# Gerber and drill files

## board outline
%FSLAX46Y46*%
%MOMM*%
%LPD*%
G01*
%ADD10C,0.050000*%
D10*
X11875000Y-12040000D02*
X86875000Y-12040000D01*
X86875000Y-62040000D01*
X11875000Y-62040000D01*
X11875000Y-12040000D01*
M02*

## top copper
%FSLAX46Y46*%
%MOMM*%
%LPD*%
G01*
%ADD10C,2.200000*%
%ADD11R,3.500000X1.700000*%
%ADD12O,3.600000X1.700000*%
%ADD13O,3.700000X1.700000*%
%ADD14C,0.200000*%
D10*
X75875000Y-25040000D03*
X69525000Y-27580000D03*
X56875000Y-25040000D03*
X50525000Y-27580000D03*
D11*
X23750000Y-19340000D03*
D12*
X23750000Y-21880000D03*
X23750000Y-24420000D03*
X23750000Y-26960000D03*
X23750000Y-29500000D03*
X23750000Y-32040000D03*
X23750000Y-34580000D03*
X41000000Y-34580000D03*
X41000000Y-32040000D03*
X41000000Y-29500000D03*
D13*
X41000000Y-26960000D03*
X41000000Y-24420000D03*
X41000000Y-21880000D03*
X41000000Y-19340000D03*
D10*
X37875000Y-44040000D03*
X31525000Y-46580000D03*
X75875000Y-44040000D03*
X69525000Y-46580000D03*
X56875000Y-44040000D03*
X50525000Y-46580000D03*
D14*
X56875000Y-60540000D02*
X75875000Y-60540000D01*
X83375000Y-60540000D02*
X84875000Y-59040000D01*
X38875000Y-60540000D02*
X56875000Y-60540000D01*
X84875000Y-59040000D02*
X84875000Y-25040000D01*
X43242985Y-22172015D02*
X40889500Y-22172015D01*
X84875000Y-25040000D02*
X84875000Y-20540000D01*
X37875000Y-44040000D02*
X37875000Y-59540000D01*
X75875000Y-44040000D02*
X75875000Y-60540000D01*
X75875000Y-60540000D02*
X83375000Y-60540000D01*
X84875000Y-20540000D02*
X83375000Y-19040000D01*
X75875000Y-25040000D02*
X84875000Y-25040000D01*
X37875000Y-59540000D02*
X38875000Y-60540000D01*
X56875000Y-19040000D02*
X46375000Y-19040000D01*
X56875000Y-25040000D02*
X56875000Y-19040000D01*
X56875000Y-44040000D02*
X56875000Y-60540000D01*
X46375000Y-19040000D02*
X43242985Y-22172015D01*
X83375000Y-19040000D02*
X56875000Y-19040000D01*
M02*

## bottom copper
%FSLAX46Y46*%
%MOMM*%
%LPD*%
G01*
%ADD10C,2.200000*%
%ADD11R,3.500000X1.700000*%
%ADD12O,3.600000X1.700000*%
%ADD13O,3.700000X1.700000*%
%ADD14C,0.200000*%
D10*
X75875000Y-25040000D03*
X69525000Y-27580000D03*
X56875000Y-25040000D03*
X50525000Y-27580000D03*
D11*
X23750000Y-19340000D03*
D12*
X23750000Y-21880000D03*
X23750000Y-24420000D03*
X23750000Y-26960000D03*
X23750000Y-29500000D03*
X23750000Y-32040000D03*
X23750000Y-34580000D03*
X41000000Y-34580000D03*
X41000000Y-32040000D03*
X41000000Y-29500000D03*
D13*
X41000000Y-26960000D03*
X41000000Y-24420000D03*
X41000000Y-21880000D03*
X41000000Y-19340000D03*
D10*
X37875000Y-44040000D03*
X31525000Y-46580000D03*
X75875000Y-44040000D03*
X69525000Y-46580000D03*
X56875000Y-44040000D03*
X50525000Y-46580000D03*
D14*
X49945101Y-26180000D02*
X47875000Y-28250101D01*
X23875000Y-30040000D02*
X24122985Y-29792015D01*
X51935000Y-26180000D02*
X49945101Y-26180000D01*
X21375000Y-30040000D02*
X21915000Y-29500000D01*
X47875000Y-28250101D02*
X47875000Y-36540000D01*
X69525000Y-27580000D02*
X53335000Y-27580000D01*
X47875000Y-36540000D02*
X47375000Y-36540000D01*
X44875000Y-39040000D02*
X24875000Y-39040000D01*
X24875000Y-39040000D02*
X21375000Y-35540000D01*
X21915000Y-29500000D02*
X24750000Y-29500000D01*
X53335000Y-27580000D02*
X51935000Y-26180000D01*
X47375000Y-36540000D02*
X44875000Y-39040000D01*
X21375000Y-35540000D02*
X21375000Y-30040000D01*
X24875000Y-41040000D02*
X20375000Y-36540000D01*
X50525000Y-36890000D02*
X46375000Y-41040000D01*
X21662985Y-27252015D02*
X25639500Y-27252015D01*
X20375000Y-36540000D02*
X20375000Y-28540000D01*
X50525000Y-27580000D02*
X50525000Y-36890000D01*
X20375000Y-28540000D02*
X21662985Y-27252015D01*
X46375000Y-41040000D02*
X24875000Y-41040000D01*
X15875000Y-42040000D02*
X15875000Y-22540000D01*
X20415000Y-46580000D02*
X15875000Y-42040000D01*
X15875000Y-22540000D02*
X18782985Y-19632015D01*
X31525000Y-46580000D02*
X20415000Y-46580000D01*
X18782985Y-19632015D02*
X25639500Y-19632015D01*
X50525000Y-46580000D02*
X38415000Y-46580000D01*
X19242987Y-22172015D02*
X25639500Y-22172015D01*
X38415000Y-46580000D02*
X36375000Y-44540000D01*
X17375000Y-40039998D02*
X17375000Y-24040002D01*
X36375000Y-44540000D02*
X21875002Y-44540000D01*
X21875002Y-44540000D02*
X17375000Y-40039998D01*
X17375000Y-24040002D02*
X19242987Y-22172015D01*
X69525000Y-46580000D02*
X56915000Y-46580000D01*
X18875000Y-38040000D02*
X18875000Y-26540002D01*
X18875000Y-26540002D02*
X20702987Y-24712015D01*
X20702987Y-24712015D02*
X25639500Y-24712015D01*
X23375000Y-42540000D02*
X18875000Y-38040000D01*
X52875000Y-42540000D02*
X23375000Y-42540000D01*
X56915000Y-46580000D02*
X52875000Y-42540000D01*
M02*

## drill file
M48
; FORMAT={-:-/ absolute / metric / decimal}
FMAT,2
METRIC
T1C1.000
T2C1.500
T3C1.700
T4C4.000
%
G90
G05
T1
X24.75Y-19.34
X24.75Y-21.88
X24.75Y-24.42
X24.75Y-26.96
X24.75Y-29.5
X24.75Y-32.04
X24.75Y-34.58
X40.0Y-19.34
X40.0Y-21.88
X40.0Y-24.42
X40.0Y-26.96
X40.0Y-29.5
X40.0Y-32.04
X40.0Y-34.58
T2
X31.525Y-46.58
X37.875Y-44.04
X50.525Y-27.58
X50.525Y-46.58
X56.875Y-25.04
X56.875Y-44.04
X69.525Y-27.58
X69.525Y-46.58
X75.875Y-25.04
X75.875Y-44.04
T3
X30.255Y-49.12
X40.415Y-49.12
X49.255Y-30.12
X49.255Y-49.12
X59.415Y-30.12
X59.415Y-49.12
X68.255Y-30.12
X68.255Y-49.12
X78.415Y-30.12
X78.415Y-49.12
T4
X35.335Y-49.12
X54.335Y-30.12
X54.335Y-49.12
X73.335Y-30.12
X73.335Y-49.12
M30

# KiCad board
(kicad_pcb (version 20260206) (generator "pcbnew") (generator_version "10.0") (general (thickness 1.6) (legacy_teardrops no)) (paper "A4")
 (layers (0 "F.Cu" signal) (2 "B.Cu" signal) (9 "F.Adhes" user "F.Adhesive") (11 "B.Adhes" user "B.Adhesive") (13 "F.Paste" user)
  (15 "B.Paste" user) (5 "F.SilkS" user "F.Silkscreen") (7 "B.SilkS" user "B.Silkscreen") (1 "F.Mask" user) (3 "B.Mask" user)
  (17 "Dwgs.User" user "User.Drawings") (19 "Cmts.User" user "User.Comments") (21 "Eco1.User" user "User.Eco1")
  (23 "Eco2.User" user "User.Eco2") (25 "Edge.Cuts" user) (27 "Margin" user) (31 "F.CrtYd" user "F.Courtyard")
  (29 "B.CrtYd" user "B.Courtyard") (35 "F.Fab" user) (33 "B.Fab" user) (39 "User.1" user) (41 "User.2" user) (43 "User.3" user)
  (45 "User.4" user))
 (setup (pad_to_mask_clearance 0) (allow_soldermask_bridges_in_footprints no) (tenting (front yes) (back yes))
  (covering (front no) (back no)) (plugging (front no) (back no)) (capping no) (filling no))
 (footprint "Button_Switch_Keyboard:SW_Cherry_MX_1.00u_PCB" (layer "F.Cu") (at 75.875 25.04)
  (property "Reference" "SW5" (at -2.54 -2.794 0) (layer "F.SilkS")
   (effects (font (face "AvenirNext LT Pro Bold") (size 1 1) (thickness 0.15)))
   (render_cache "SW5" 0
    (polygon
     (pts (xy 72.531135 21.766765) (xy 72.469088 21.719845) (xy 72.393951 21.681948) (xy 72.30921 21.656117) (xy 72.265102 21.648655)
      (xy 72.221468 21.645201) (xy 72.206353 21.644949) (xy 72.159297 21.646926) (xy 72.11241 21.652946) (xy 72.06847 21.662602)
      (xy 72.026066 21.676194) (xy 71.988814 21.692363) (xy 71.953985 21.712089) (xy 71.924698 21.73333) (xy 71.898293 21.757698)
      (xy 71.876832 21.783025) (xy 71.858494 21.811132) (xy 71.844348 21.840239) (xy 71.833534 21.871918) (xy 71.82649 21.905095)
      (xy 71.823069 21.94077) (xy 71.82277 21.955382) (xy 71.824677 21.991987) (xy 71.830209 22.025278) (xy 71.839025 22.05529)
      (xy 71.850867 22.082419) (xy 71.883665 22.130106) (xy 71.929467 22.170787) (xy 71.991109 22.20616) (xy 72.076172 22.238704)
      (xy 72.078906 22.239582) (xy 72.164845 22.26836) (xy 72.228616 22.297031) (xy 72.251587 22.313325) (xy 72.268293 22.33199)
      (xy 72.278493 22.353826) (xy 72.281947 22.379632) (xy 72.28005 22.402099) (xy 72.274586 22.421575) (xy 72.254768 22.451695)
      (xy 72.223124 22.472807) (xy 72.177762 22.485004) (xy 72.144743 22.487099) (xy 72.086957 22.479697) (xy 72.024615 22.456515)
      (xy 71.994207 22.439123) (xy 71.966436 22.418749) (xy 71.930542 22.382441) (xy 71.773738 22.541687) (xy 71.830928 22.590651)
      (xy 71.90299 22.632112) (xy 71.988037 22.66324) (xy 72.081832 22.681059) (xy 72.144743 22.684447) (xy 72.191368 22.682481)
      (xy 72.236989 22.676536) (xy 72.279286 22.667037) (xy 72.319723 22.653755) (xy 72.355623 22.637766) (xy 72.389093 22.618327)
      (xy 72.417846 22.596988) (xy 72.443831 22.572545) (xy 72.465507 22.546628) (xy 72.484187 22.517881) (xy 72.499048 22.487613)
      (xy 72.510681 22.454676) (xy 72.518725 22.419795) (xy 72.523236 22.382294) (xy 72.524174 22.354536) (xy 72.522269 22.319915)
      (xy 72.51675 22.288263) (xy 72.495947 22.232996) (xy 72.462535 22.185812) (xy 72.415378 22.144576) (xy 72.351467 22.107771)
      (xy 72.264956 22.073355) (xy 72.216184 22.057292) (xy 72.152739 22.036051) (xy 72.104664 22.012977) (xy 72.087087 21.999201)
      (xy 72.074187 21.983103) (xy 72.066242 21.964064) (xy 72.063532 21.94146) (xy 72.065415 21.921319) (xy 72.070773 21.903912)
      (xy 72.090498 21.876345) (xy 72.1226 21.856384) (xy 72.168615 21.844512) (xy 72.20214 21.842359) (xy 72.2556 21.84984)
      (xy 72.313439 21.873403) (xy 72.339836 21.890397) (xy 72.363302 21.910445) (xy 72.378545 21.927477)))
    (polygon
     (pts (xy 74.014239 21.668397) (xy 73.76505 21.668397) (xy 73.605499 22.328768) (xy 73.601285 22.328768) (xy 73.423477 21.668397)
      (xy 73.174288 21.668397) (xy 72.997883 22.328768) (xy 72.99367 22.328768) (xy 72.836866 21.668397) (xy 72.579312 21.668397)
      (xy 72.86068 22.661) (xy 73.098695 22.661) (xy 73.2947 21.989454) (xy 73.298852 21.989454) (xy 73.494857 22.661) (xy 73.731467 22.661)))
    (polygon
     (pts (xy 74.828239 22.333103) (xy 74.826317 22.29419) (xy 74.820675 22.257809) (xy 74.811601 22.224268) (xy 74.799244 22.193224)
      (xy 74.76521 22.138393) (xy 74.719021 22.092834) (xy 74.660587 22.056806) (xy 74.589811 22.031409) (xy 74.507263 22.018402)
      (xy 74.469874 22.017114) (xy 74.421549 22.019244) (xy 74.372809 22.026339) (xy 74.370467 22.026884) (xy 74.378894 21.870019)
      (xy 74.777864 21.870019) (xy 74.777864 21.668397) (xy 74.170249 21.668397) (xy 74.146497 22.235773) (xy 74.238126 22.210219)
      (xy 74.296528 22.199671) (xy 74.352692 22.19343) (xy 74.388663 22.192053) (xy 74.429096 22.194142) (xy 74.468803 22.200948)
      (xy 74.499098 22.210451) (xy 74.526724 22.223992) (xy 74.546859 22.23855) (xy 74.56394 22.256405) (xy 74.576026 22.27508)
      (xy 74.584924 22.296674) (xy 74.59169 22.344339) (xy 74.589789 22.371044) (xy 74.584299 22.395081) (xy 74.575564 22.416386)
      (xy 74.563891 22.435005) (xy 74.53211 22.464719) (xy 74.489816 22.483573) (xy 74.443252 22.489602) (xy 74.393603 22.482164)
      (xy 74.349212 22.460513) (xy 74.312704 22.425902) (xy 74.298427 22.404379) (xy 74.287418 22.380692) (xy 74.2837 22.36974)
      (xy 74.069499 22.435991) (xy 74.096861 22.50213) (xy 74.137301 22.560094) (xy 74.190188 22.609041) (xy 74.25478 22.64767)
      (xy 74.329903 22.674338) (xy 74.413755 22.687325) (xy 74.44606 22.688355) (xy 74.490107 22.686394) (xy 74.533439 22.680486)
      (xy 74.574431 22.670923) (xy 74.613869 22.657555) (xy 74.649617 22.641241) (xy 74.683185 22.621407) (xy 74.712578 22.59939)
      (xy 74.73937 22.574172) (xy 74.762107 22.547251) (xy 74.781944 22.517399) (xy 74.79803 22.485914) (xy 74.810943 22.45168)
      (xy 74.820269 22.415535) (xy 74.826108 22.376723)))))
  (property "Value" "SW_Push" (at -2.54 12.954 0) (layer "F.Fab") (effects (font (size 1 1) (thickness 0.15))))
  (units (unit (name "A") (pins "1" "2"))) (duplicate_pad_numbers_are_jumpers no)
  (pad "" np_thru_hole circle (at -7.62 5.08) (size 1.7 1.7) (drill 1.7) (layers "*.Cu" "*.Mask"))
  (pad "" np_thru_hole circle (at -2.54 5.08) (size 4 4) (drill 4) (layers "*.Cu" "*.Mask"))
  (pad "" np_thru_hole circle (at 2.54 5.08) (size 1.7 1.7) (drill 1.7) (layers "*.Cu" "*.Mask"))
  (pad "1" thru_hole circle (at 0 0) (size 2.2 2.2) (drill 1.5) (layers "*.Cu" "*.Mask") (remove_unused_layers no) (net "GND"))
  (pad "2" thru_hole circle (at -6.35 2.54) (size 2.2 2.2) (drill 1.5) (layers "*.Cu" "*.Mask") (remove_unused_layers no)
   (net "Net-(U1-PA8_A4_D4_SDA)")))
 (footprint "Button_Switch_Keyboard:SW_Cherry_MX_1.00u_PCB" (layer "F.Cu") (at 56.875 25.04)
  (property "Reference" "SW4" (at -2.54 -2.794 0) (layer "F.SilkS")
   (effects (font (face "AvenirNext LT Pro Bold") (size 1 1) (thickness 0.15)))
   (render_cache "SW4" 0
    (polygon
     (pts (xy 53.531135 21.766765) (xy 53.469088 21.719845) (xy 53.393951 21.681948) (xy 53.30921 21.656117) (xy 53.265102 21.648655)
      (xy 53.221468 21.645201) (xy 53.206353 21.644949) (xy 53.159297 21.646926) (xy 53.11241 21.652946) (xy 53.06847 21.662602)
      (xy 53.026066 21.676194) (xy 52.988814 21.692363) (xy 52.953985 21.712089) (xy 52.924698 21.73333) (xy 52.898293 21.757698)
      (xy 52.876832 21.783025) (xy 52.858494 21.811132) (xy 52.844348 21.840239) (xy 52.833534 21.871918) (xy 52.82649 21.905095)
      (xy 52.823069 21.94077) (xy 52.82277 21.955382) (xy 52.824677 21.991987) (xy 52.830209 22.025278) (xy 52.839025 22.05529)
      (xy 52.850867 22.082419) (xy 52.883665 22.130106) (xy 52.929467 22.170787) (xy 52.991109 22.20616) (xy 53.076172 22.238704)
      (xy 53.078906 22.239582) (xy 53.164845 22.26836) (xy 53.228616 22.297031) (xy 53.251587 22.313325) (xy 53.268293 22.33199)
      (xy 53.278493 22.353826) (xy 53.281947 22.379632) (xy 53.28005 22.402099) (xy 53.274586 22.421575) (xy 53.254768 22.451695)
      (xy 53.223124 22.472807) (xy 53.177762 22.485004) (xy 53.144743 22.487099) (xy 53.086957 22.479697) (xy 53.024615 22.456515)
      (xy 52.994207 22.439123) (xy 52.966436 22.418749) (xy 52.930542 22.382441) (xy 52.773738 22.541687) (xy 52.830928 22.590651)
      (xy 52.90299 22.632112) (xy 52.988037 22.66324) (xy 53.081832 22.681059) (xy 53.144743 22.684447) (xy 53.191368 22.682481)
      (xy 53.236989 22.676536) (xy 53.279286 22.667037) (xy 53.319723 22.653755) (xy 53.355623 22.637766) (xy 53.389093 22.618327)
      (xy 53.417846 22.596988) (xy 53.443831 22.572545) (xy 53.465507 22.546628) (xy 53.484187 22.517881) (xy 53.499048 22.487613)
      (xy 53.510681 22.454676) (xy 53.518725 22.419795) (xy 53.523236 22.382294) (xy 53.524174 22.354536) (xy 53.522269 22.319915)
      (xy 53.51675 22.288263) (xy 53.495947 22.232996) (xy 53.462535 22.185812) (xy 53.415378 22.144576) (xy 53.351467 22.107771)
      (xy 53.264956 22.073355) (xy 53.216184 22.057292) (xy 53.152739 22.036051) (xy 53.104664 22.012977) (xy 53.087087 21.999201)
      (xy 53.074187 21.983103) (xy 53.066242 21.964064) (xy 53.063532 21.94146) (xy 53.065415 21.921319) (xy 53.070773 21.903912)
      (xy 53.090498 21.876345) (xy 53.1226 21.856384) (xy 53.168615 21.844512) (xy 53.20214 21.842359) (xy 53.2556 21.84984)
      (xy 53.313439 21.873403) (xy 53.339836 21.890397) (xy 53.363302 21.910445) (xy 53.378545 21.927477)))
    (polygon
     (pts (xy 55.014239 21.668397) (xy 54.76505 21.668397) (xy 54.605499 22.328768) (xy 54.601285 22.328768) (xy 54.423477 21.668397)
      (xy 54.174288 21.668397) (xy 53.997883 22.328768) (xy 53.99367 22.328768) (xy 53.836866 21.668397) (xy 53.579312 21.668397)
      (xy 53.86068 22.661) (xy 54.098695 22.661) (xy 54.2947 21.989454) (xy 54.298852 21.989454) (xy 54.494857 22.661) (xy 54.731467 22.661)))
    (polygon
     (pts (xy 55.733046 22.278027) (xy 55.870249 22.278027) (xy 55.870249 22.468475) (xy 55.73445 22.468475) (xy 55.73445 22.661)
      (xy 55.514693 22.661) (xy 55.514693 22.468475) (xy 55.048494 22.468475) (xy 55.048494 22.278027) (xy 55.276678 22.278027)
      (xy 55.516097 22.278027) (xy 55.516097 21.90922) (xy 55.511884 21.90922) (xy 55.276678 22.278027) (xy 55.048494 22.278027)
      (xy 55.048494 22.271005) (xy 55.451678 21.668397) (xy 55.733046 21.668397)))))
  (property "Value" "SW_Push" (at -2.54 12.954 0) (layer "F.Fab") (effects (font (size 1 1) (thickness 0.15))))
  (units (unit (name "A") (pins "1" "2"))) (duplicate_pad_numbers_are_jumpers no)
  (pad "" np_thru_hole circle (at -7.62 5.08) (size 1.7 1.7) (drill 1.7) (layers "*.Cu" "*.Mask"))
  (pad "" np_thru_hole circle (at -2.54 5.08) (size 4 4) (drill 4) (layers "*.Cu" "*.Mask"))
  (pad "" np_thru_hole circle (at 2.54 5.08) (size 1.7 1.7) (drill 1.7) (layers "*.Cu" "*.Mask"))
  (pad "1" thru_hole circle (at 0 0) (size 2.2 2.2) (drill 1.5) (layers "*.Cu" "*.Mask") (remove_unused_layers no) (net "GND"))
  (pad "2" thru_hole circle (at -6.35 2.54) (size 2.2 2.2) (drill 1.5) (layers "*.Cu" "*.Mask") (remove_unused_layers no)
   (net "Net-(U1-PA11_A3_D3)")))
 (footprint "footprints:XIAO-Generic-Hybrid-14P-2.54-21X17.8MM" (layer "F.Cu") (at 32.375 26.96)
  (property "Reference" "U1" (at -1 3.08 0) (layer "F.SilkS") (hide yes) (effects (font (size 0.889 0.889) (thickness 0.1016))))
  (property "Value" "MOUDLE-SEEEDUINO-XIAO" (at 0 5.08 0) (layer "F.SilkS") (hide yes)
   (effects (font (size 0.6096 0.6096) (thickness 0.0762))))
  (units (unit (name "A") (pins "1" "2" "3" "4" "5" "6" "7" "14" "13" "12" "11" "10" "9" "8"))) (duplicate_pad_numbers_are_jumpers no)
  (pad "1" thru_hole rect (at -7.625 -7.62) (size 3.5 1.7) (drill 1 (offset -1 0)) (layers "*.Cu" "*.Mask") (remove_unused_layers no)
   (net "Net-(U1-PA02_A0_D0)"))
  (pad "2" thru_hole oval (at -7.625 -5.08) (size 3.6 1.7) (drill 1 (offset -1 0)) (layers "*.Cu" "*.Mask") (remove_unused_layers no)
   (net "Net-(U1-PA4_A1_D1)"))
  (pad "3" thru_hole oval (at -7.625 -2.54) (size 3.6 1.7) (drill 1 (offset -1 0)) (layers "*.Cu" "*.Mask") (remove_unused_layers no)
   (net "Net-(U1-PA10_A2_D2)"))
  (pad "4" thru_hole oval (at -7.625 0) (size 3.6 1.7) (drill 1 (offset -1 0)) (layers "*.Cu" "*.Mask") (remove_unused_layers no)
   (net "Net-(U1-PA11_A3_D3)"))
  (pad "5" thru_hole oval (at -7.625 2.54) (size 3.6 1.7) (drill 1 (offset -1 0)) (layers "*.Cu" "*.Mask") (remove_unused_layers no)
   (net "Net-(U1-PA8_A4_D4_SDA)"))
  (pad "6" thru_hole oval (at -7.625 5.08 180) (size 3.6 1.7) (drill 1 (offset 1 0)) (layers "*.Cu" "*.Mask") (remove_unused_layers no)
   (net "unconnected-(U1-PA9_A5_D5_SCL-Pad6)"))
  (pad "7" thru_hole oval (at -7.625 7.62) (size 3.6 1.7) (drill 1 (offset -1 0)) (layers "*.Cu" "*.Mask") (remove_unused_layers no)
   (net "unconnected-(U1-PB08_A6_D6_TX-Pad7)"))
  (pad "8" thru_hole oval (at 7.625 7.62) (size 3.6 1.7) (drill 1 (offset 1 0)) (layers "*.Cu" "*.Mask") (remove_unused_layers no)
   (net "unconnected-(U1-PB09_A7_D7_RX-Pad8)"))
  (pad "9" thru_hole oval (at 7.625 5.08) (size 3.6 1.7) (drill 1 (offset 1 0)) (layers "*.Cu" "*.Mask") (remove_unused_layers no)
   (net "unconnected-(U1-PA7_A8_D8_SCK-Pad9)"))
  (pad "10" thru_hole oval (at 7.625 2.54) (size 3.6 1.7) (drill 1 (offset 1 0)) (layers "*.Cu" "*.Mask") (remove_unused_layers no)
   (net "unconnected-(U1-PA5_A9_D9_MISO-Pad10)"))
  (pad "11" thru_hole oval (at 7.625 0) (size 3.7 1.7) (drill 1 (offset 1 0)) (layers "*.Cu" "*.Mask") (remove_unused_layers no)
   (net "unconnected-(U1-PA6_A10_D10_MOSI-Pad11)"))
  (pad "12" thru_hole oval (at 7.625 -2.54) (size 3.7 1.7) (drill 1 (offset 1 0)) (layers "*.Cu" "*.Mask") (remove_unused_layers no)
   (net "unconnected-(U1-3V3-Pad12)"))
  (pad "13" thru_hole oval (at 7.625 -5.08) (size 3.7 1.7) (drill 1 (offset 1 0)) (layers "*.Cu" "*.Mask") (remove_unused_layers no)
   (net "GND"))
  (pad "14" thru_hole oval (at 7.625 -7.62) (size 3.7 1.7) (drill 1 (offset 1 0)) (layers "*.Cu" "*.Mask") (remove_unused_layers no)
   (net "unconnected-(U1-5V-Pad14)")))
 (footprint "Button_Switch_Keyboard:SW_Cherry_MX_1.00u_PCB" (layer "F.Cu") (at 37.875 44.04)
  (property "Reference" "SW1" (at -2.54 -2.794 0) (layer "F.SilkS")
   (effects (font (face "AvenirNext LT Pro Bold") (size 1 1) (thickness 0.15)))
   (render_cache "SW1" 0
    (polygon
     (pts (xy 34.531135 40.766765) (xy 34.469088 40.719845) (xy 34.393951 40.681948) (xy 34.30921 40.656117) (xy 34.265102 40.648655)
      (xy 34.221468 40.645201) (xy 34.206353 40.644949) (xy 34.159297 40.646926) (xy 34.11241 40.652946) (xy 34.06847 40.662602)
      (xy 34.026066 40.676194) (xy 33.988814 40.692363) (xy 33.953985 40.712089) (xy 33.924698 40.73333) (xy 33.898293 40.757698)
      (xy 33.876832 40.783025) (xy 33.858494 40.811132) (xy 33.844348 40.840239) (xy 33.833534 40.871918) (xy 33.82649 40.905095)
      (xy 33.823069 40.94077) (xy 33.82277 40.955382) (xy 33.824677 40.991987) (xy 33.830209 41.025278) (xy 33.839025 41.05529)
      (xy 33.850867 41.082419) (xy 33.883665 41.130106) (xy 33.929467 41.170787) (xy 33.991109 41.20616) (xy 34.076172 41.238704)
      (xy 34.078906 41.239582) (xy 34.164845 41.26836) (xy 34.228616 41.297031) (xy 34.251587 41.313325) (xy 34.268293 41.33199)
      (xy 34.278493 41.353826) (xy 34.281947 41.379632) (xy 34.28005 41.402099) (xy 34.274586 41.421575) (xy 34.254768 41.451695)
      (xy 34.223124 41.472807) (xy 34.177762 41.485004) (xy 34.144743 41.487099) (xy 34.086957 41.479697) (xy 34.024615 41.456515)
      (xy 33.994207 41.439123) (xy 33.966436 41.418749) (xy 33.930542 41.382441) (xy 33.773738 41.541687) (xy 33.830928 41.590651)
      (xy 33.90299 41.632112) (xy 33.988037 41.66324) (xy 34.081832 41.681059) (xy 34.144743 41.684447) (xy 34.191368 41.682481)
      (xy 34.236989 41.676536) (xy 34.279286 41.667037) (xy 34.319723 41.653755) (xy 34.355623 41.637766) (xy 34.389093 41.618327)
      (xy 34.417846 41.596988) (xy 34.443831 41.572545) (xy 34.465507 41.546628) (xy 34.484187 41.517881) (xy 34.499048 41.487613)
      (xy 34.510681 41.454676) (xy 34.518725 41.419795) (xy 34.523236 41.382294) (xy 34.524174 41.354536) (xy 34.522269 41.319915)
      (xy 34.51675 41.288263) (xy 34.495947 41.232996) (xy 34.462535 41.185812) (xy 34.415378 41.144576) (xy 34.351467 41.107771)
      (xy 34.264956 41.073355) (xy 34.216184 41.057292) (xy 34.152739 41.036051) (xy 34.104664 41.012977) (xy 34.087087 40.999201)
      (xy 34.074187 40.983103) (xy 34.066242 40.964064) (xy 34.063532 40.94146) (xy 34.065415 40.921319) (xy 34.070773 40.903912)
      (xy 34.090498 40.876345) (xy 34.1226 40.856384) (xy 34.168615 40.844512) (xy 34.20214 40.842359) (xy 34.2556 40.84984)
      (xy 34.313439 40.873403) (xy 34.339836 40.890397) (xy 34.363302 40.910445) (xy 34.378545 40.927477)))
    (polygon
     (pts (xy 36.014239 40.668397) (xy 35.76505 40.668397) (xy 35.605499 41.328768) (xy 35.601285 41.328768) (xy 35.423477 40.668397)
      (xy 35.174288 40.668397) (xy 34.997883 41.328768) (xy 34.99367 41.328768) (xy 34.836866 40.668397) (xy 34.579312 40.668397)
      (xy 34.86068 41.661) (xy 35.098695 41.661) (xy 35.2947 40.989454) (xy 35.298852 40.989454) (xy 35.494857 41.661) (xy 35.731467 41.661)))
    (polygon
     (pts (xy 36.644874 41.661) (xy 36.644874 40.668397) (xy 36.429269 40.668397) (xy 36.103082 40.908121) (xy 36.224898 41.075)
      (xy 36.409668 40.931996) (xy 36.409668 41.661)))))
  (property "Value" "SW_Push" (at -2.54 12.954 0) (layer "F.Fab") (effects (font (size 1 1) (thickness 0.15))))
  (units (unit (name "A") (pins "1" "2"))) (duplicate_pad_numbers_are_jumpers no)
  (pad "" np_thru_hole circle (at -7.62 5.08) (size 1.7 1.7) (drill 1.7) (layers "*.Cu" "*.Mask"))
  (pad "" np_thru_hole circle (at -2.54 5.08) (size 4 4) (drill 4) (layers "*.Cu" "*.Mask"))
  (pad "" np_thru_hole circle (at 2.54 5.08) (size 1.7 1.7) (drill 1.7) (layers "*.Cu" "*.Mask"))
  (pad "1" thru_hole circle (at 0 0) (size 2.2 2.2) (drill 1.5) (layers "*.Cu" "*.Mask") (remove_unused_layers no) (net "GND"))
  (pad "2" thru_hole circle (at -6.35 2.54) (size 2.2 2.2) (drill 1.5) (layers "*.Cu" "*.Mask") (remove_unused_layers no)
   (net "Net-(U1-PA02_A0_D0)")))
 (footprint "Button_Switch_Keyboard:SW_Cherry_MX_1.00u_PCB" (layer "F.Cu") (at 75.875 44.04)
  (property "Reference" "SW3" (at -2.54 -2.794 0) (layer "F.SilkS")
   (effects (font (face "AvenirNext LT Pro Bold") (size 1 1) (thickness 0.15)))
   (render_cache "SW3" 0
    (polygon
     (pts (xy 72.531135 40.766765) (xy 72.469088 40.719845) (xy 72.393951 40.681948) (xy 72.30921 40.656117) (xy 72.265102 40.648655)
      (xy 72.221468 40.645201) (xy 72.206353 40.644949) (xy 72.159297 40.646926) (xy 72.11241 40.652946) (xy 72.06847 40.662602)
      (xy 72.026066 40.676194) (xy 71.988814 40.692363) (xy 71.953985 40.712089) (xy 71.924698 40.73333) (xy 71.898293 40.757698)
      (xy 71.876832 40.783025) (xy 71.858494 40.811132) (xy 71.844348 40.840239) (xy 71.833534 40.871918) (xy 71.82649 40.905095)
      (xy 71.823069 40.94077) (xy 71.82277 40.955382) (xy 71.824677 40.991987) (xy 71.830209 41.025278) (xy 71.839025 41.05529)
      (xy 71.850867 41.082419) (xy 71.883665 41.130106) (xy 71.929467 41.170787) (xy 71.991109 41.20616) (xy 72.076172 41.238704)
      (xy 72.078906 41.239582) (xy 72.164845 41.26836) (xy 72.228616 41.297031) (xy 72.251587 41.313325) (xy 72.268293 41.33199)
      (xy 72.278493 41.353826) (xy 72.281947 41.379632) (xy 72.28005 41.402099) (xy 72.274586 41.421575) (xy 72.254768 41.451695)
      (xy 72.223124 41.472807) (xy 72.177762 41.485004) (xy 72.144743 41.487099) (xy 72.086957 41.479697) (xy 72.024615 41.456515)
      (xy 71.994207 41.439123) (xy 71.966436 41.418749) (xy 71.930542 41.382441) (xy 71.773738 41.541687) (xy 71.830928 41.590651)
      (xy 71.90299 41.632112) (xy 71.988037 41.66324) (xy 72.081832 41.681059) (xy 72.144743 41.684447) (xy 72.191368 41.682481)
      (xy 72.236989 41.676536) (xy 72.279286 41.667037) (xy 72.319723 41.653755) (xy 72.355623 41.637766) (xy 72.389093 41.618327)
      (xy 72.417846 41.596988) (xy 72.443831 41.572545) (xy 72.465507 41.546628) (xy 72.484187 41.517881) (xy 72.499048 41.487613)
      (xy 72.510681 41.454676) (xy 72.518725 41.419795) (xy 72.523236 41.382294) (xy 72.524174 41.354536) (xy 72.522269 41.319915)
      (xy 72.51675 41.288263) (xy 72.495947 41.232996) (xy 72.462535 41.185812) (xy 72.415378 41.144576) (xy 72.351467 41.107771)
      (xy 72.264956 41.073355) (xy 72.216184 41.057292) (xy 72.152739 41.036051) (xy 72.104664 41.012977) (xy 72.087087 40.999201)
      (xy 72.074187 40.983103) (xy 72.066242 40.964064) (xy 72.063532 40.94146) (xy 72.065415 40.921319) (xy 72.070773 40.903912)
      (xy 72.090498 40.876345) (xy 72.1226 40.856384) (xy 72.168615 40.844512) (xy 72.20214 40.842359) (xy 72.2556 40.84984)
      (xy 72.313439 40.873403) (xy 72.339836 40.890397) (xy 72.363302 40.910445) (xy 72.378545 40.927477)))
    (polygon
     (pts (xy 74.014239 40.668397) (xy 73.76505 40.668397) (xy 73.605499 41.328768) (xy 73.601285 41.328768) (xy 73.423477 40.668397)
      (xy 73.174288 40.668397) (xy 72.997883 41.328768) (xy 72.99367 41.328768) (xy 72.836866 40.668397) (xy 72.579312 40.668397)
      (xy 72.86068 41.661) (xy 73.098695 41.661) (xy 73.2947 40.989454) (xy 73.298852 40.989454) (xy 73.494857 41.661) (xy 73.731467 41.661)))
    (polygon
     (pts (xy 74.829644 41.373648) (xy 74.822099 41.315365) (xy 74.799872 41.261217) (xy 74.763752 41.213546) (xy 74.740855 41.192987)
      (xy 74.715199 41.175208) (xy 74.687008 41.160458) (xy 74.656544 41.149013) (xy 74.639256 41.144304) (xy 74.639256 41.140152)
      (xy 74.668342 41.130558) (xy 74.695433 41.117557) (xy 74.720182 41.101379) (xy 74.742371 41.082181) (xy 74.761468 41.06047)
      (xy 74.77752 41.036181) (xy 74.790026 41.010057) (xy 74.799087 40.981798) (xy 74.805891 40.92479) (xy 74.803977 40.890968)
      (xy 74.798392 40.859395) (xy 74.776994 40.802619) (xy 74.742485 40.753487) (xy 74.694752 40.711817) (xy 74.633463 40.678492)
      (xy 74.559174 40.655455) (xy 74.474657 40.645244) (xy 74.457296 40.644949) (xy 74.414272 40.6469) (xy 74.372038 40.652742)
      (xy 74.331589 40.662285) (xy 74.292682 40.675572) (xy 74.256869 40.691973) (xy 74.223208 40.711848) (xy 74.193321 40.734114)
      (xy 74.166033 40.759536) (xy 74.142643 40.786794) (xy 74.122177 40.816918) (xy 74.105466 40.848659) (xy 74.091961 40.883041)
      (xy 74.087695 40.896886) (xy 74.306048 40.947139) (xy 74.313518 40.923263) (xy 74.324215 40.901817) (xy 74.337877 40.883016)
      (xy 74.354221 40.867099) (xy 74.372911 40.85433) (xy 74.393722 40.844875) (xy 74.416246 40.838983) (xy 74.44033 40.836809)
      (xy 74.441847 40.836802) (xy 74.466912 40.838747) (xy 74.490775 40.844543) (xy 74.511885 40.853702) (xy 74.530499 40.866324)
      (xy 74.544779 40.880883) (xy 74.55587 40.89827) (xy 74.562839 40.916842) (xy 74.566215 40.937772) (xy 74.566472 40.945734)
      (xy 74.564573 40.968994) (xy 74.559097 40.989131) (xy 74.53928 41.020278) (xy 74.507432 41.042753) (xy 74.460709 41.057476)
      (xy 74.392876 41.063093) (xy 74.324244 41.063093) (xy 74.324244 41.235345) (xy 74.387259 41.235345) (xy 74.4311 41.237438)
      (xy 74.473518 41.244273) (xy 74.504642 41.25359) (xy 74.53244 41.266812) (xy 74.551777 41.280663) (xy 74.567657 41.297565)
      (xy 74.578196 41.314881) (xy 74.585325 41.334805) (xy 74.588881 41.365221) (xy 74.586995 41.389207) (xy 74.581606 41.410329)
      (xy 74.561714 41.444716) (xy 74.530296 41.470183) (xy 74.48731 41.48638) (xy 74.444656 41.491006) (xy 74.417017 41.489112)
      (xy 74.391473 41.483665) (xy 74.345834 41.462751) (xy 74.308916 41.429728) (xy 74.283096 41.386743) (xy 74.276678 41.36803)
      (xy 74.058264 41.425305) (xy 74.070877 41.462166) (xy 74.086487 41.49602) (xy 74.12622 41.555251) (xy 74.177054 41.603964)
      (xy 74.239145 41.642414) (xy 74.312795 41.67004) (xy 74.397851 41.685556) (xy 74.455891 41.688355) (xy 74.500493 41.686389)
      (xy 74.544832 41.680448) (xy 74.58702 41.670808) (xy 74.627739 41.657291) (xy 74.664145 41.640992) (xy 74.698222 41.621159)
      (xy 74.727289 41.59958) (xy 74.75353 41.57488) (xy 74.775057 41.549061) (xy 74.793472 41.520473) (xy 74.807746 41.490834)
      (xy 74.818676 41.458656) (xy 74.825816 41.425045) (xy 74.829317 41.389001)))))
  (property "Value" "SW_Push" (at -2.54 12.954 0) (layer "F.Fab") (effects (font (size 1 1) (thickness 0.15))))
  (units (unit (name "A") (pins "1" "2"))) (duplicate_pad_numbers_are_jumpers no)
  (pad "" np_thru_hole circle (at -7.62 5.08) (size 1.7 1.7) (drill 1.7) (layers "*.Cu" "*.Mask"))
  (pad "" np_thru_hole circle (at -2.54 5.08) (size 4 4) (drill 4) (layers "*.Cu" "*.Mask"))
  (pad "" np_thru_hole circle (at 2.54 5.08) (size 1.7 1.7) (drill 1.7) (layers "*.Cu" "*.Mask"))
  (pad "1" thru_hole circle (at 0 0) (size 2.2 2.2) (drill 1.5) (layers "*.Cu" "*.Mask") (remove_unused_layers no) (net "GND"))
  (pad "2" thru_hole circle (at -6.35 2.54) (size 2.2 2.2) (drill 1.5) (layers "*.Cu" "*.Mask") (remove_unused_layers no)
   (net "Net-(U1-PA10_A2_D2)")))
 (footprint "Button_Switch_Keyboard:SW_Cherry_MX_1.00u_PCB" (layer "F.Cu") (at 56.875 44.04)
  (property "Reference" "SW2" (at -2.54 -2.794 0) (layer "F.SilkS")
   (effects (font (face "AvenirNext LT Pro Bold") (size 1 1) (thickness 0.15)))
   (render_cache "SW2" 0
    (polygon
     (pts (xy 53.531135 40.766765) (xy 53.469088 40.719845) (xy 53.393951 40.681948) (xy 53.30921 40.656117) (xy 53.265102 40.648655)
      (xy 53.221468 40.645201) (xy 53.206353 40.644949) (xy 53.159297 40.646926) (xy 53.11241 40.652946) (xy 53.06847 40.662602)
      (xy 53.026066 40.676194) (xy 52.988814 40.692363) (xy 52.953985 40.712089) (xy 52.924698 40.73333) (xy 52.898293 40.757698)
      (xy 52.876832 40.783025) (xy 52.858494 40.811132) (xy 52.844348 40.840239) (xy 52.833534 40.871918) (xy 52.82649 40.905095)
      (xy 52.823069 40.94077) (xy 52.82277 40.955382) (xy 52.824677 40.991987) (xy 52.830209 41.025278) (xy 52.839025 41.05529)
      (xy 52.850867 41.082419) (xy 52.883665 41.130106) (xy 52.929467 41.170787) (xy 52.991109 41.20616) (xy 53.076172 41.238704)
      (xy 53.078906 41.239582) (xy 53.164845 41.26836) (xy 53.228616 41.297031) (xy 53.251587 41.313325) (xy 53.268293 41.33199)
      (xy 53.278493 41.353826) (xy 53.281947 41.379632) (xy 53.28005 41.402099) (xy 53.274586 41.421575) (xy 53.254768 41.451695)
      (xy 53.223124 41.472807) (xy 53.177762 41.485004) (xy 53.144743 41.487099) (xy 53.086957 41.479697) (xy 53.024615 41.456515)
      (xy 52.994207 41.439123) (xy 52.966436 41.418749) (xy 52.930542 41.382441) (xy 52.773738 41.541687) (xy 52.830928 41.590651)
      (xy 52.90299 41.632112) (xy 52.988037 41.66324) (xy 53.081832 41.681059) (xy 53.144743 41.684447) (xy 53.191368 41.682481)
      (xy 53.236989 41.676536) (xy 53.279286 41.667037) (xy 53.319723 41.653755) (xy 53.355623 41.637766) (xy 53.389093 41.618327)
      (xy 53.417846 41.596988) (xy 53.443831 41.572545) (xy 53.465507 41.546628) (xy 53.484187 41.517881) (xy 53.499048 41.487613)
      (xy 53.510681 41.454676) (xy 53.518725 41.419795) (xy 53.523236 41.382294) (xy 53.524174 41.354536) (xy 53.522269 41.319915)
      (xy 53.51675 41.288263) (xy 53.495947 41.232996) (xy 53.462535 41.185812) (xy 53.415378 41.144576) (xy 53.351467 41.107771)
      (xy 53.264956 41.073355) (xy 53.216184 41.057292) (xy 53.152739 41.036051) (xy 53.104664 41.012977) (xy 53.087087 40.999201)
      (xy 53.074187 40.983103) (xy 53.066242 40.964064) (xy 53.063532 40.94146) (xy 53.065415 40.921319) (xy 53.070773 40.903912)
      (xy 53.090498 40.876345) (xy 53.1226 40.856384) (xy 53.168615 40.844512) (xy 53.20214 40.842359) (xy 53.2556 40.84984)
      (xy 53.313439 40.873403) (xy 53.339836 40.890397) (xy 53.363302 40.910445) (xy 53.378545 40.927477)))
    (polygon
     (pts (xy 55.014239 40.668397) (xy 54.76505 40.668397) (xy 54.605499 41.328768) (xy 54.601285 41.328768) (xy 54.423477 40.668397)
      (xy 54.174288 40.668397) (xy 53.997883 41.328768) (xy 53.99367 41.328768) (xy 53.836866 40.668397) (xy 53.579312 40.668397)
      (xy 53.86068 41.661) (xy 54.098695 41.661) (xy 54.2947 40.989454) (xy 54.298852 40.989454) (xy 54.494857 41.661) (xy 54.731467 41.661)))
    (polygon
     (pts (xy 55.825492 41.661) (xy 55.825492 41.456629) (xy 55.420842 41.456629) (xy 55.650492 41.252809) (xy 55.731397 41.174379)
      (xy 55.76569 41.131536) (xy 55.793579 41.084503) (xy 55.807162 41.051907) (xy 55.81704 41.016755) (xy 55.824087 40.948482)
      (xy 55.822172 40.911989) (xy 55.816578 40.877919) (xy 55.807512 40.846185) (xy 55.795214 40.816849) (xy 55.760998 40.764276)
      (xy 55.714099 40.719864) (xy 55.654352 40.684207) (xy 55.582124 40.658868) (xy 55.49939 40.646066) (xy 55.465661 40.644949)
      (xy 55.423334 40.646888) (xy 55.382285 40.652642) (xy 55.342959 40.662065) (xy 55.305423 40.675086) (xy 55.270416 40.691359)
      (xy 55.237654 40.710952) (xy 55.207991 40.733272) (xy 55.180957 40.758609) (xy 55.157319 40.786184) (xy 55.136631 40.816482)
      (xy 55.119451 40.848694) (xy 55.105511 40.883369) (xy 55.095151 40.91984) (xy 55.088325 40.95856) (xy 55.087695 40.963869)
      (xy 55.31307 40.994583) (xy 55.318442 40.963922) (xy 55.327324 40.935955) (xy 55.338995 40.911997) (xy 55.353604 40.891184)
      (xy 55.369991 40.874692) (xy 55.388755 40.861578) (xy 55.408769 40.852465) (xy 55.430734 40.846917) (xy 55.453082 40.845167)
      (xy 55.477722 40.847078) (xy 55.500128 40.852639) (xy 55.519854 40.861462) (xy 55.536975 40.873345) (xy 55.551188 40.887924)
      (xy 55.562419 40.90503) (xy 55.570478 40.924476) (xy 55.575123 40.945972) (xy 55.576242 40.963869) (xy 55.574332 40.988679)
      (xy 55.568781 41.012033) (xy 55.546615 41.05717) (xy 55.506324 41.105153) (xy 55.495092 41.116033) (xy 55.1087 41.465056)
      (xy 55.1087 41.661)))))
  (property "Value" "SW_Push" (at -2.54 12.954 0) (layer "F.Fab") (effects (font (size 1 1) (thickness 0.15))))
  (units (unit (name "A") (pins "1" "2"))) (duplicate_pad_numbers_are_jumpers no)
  (pad "" np_thru_hole circle (at -7.62 5.08) (size 1.7 1.7) (drill 1.7) (layers "*.Cu" "*.Mask"))
  (pad "" np_thru_hole circle (at -2.54 5.08) (size 4 4) (drill 4) (layers "*.Cu" "*.Mask"))
  (pad "" np_thru_hole circle (at 2.54 5.08) (size 1.7 1.7) (drill 1.7) (layers "*.Cu" "*.Mask"))
  (pad "1" thru_hole circle (at 0 0) (size 2.2 2.2) (drill 1.5) (layers "*.Cu" "*.Mask") (remove_unused_layers no) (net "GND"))
  (pad "2" thru_hole circle (at -6.35 2.54) (size 2.2 2.2) (drill 1.5) (layers "*.Cu" "*.Mask") (remove_unused_layers no)
   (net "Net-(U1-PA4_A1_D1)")))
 (gr_rect (start 11.875 12.04) (end 86.875 62.04) (stroke (width 0.05) (type default)) (fill no) (layer "Edge.Cuts"))
 (segment (start 56.875 60.54) (end 75.875 60.54) (width 0.2) (layer "F.Cu") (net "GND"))
 (segment (start 83.375 60.54) (end 84.875 59.04) (width 0.2) (layer "F.Cu") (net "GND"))
 (segment (start 38.875 60.54) (end 56.875 60.54) (width 0.2) (layer "F.Cu") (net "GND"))
 (segment (start 84.875 59.04) (end 84.875 25.04) (width 0.2) (layer "F.Cu") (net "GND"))
 (segment (start 43.242985 22.172015) (end 40.8895 22.172015) (width 0.2) (layer "F.Cu") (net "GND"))
 (segment (start 84.875 25.04) (end 84.875 20.54) (width 0.2) (layer "F.Cu") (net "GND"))
 (segment (start 37.875 44.04) (end 37.875 59.54) (width 0.2) (layer "F.Cu") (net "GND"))
 (segment (start 75.875 44.04) (end 75.875 60.54) (width 0.2) (layer "F.Cu") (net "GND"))
 (segment (start 75.875 60.54) (end 83.375 60.54) (width 0.2) (layer "F.Cu") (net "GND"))
 (segment (start 84.875 20.54) (end 83.375 19.04) (width 0.2) (layer "F.Cu") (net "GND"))
 (segment (start 75.875 25.04) (end 84.875 25.04) (width 0.2) (layer "F.Cu") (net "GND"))
 (segment (start 37.875 59.54) (end 38.875 60.54) (width 0.2) (layer "F.Cu") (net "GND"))
 (segment (start 56.875 19.04) (end 46.375 19.04) (width 0.2) (layer "F.Cu") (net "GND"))
 (segment (start 56.875 25.04) (end 56.875 19.04) (width 0.2) (layer "F.Cu") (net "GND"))
 (segment (start 56.875 44.04) (end 56.875 60.54) (width 0.2) (layer "F.Cu") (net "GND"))
 (segment (start 46.375 19.04) (end 43.242985 22.172015) (width 0.2) (layer "F.Cu") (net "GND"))
 (segment (start 83.375 19.04) (end 56.875 19.04) (width 0.2) (layer "F.Cu") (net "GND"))
 (segment (start 49.945101 26.18) (end 47.875 28.250101) (width 0.2) (layer "B.Cu") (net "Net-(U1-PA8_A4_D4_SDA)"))
 (segment (start 23.875 30.04) (end 24.122985 29.792015) (width 0.2) (layer "B.Cu") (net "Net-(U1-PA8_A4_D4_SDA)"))
 (segment (start 51.935 26.18) (end 49.945101 26.18) (width 0.2) (layer "B.Cu") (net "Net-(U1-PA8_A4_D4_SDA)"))
 (segment (start 21.375 30.04) (end 21.915 29.5) (width 0.2) (layer "B.Cu") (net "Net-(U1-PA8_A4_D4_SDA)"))
 (segment (start 47.875 28.250101) (end 47.875 36.54) (width 0.2) (layer "B.Cu") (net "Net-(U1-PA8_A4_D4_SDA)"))
 (segment (start 69.525 27.58) (end 53.335 27.58) (width 0.2) (layer "B.Cu") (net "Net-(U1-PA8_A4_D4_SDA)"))
 (segment (start 47.875 36.54) (end 47.375 36.54) (width 0.2) (layer "B.Cu") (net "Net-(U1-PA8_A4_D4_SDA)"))
 (segment (start 44.875 39.04) (end 24.875 39.04) (width 0.2) (layer "B.Cu") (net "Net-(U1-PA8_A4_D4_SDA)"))
 (segment (start 24.875 39.04) (end 21.375 35.54) (width 0.2) (layer "B.Cu") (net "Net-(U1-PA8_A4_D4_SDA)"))
 (segment (start 21.915 29.5) (end 24.75 29.5) (width 0.2) (layer "B.Cu") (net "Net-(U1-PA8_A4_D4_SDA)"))
 (segment (start 53.335 27.58) (end 51.935 26.18) (width 0.2) (layer "B.Cu") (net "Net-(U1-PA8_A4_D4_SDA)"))
 (segment (start 47.375 36.54) (end 44.875 39.04) (width 0.2) (layer "B.Cu") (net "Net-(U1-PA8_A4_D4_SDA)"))
 (segment (start 21.375 35.54) (end 21.375 30.04) (width 0.2) (layer "B.Cu") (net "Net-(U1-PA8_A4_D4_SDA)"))
 (segment (start 24.875 41.04) (end 20.375 36.54) (width 0.2) (layer "B.Cu") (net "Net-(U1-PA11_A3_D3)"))
 (segment (start 50.525 36.89) (end 46.375 41.04) (width 0.2) (layer "B.Cu") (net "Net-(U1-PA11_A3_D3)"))
 (segment (start 21.662985 27.252015) (end 25.6395 27.252015) (width 0.2) (layer "B.Cu") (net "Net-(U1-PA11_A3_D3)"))
 (segment (start 20.375 36.54) (end 20.375 28.54) (width 0.2) (layer "B.Cu") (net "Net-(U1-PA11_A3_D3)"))
 (segment (start 50.525 27.58) (end 50.525 36.89) (width 0.2) (layer "B.Cu") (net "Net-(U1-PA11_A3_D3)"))
 (segment (start 20.375 28.54) (end 21.662985 27.252015) (width 0.2) (layer "B.Cu") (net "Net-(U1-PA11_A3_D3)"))
 (segment (start 46.375 41.04) (end 24.875 41.04) (width 0.2) (layer "B.Cu") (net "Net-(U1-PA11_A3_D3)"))
 (segment (start 15.875 42.04) (end 15.875 22.54) (width 0.2) (layer "B.Cu") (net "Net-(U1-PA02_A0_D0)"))
 (segment (start 20.415 46.58) (end 15.875 42.04) (width 0.2) (layer "B.Cu") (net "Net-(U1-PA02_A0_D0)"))
 (segment (start 15.875 22.54) (end 18.782985 19.632015) (width 0.2) (layer "B.Cu") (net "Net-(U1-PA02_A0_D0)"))
 (segment (start 31.525 46.58) (end 20.415 46.58) (width 0.2) (layer "B.Cu") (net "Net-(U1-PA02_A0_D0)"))
 (segment (start 18.782985 19.632015) (end 25.6395 19.632015) (width 0.2) (layer "B.Cu") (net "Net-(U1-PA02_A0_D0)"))
 (segment (start 50.525 46.58) (end 38.415 46.58) (width 0.2) (layer "B.Cu") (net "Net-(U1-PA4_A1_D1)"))
 (segment (start 19.242987 22.172015) (end 25.6395 22.172015) (width 0.2) (layer "B.Cu") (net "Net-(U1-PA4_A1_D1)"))
 (segment (start 38.415 46.58) (end 36.375 44.54) (width 0.2) (layer "B.Cu") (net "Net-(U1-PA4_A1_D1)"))
 (segment (start 17.375 40.039998) (end 17.375 24.040002) (width 0.2) (layer "B.Cu") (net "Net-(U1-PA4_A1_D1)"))
 (segment (start 36.375 44.54) (end 21.875002 44.54) (width 0.2) (layer "B.Cu") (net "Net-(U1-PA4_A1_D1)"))
 (segment (start 21.875002 44.54) (end 17.375 40.039998) (width 0.2) (layer "B.Cu") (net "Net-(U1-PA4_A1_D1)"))
 (segment (start 17.375 24.040002) (end 19.242987 22.172015) (width 0.2) (layer "B.Cu") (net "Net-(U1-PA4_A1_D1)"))
 (segment (start 69.525 46.58) (end 56.915 46.58) (width 0.2) (layer "B.Cu") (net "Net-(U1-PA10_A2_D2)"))
 (segment (start 18.875 38.04) (end 18.875 26.540002) (width 0.2) (layer "B.Cu") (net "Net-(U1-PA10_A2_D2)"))
 (segment (start 18.875 26.540002) (end 20.702987 24.712015) (width 0.2) (layer "B.Cu") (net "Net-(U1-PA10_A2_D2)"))
 (segment (start 20.702987 24.712015) (end 25.6395 24.712015) (width 0.2) (layer "B.Cu") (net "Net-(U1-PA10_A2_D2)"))
 (segment (start 23.375 42.54) (end 18.875 38.04) (width 0.2) (layer "B.Cu") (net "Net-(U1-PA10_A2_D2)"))
 (segment (start 52.875 42.54) (end 23.375 42.54) (width 0.2) (layer "B.Cu") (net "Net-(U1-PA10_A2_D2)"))
 (segment (start 56.915 46.58) (end 52.875 42.54) (width 0.2) (layer "B.Cu") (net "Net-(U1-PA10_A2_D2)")))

